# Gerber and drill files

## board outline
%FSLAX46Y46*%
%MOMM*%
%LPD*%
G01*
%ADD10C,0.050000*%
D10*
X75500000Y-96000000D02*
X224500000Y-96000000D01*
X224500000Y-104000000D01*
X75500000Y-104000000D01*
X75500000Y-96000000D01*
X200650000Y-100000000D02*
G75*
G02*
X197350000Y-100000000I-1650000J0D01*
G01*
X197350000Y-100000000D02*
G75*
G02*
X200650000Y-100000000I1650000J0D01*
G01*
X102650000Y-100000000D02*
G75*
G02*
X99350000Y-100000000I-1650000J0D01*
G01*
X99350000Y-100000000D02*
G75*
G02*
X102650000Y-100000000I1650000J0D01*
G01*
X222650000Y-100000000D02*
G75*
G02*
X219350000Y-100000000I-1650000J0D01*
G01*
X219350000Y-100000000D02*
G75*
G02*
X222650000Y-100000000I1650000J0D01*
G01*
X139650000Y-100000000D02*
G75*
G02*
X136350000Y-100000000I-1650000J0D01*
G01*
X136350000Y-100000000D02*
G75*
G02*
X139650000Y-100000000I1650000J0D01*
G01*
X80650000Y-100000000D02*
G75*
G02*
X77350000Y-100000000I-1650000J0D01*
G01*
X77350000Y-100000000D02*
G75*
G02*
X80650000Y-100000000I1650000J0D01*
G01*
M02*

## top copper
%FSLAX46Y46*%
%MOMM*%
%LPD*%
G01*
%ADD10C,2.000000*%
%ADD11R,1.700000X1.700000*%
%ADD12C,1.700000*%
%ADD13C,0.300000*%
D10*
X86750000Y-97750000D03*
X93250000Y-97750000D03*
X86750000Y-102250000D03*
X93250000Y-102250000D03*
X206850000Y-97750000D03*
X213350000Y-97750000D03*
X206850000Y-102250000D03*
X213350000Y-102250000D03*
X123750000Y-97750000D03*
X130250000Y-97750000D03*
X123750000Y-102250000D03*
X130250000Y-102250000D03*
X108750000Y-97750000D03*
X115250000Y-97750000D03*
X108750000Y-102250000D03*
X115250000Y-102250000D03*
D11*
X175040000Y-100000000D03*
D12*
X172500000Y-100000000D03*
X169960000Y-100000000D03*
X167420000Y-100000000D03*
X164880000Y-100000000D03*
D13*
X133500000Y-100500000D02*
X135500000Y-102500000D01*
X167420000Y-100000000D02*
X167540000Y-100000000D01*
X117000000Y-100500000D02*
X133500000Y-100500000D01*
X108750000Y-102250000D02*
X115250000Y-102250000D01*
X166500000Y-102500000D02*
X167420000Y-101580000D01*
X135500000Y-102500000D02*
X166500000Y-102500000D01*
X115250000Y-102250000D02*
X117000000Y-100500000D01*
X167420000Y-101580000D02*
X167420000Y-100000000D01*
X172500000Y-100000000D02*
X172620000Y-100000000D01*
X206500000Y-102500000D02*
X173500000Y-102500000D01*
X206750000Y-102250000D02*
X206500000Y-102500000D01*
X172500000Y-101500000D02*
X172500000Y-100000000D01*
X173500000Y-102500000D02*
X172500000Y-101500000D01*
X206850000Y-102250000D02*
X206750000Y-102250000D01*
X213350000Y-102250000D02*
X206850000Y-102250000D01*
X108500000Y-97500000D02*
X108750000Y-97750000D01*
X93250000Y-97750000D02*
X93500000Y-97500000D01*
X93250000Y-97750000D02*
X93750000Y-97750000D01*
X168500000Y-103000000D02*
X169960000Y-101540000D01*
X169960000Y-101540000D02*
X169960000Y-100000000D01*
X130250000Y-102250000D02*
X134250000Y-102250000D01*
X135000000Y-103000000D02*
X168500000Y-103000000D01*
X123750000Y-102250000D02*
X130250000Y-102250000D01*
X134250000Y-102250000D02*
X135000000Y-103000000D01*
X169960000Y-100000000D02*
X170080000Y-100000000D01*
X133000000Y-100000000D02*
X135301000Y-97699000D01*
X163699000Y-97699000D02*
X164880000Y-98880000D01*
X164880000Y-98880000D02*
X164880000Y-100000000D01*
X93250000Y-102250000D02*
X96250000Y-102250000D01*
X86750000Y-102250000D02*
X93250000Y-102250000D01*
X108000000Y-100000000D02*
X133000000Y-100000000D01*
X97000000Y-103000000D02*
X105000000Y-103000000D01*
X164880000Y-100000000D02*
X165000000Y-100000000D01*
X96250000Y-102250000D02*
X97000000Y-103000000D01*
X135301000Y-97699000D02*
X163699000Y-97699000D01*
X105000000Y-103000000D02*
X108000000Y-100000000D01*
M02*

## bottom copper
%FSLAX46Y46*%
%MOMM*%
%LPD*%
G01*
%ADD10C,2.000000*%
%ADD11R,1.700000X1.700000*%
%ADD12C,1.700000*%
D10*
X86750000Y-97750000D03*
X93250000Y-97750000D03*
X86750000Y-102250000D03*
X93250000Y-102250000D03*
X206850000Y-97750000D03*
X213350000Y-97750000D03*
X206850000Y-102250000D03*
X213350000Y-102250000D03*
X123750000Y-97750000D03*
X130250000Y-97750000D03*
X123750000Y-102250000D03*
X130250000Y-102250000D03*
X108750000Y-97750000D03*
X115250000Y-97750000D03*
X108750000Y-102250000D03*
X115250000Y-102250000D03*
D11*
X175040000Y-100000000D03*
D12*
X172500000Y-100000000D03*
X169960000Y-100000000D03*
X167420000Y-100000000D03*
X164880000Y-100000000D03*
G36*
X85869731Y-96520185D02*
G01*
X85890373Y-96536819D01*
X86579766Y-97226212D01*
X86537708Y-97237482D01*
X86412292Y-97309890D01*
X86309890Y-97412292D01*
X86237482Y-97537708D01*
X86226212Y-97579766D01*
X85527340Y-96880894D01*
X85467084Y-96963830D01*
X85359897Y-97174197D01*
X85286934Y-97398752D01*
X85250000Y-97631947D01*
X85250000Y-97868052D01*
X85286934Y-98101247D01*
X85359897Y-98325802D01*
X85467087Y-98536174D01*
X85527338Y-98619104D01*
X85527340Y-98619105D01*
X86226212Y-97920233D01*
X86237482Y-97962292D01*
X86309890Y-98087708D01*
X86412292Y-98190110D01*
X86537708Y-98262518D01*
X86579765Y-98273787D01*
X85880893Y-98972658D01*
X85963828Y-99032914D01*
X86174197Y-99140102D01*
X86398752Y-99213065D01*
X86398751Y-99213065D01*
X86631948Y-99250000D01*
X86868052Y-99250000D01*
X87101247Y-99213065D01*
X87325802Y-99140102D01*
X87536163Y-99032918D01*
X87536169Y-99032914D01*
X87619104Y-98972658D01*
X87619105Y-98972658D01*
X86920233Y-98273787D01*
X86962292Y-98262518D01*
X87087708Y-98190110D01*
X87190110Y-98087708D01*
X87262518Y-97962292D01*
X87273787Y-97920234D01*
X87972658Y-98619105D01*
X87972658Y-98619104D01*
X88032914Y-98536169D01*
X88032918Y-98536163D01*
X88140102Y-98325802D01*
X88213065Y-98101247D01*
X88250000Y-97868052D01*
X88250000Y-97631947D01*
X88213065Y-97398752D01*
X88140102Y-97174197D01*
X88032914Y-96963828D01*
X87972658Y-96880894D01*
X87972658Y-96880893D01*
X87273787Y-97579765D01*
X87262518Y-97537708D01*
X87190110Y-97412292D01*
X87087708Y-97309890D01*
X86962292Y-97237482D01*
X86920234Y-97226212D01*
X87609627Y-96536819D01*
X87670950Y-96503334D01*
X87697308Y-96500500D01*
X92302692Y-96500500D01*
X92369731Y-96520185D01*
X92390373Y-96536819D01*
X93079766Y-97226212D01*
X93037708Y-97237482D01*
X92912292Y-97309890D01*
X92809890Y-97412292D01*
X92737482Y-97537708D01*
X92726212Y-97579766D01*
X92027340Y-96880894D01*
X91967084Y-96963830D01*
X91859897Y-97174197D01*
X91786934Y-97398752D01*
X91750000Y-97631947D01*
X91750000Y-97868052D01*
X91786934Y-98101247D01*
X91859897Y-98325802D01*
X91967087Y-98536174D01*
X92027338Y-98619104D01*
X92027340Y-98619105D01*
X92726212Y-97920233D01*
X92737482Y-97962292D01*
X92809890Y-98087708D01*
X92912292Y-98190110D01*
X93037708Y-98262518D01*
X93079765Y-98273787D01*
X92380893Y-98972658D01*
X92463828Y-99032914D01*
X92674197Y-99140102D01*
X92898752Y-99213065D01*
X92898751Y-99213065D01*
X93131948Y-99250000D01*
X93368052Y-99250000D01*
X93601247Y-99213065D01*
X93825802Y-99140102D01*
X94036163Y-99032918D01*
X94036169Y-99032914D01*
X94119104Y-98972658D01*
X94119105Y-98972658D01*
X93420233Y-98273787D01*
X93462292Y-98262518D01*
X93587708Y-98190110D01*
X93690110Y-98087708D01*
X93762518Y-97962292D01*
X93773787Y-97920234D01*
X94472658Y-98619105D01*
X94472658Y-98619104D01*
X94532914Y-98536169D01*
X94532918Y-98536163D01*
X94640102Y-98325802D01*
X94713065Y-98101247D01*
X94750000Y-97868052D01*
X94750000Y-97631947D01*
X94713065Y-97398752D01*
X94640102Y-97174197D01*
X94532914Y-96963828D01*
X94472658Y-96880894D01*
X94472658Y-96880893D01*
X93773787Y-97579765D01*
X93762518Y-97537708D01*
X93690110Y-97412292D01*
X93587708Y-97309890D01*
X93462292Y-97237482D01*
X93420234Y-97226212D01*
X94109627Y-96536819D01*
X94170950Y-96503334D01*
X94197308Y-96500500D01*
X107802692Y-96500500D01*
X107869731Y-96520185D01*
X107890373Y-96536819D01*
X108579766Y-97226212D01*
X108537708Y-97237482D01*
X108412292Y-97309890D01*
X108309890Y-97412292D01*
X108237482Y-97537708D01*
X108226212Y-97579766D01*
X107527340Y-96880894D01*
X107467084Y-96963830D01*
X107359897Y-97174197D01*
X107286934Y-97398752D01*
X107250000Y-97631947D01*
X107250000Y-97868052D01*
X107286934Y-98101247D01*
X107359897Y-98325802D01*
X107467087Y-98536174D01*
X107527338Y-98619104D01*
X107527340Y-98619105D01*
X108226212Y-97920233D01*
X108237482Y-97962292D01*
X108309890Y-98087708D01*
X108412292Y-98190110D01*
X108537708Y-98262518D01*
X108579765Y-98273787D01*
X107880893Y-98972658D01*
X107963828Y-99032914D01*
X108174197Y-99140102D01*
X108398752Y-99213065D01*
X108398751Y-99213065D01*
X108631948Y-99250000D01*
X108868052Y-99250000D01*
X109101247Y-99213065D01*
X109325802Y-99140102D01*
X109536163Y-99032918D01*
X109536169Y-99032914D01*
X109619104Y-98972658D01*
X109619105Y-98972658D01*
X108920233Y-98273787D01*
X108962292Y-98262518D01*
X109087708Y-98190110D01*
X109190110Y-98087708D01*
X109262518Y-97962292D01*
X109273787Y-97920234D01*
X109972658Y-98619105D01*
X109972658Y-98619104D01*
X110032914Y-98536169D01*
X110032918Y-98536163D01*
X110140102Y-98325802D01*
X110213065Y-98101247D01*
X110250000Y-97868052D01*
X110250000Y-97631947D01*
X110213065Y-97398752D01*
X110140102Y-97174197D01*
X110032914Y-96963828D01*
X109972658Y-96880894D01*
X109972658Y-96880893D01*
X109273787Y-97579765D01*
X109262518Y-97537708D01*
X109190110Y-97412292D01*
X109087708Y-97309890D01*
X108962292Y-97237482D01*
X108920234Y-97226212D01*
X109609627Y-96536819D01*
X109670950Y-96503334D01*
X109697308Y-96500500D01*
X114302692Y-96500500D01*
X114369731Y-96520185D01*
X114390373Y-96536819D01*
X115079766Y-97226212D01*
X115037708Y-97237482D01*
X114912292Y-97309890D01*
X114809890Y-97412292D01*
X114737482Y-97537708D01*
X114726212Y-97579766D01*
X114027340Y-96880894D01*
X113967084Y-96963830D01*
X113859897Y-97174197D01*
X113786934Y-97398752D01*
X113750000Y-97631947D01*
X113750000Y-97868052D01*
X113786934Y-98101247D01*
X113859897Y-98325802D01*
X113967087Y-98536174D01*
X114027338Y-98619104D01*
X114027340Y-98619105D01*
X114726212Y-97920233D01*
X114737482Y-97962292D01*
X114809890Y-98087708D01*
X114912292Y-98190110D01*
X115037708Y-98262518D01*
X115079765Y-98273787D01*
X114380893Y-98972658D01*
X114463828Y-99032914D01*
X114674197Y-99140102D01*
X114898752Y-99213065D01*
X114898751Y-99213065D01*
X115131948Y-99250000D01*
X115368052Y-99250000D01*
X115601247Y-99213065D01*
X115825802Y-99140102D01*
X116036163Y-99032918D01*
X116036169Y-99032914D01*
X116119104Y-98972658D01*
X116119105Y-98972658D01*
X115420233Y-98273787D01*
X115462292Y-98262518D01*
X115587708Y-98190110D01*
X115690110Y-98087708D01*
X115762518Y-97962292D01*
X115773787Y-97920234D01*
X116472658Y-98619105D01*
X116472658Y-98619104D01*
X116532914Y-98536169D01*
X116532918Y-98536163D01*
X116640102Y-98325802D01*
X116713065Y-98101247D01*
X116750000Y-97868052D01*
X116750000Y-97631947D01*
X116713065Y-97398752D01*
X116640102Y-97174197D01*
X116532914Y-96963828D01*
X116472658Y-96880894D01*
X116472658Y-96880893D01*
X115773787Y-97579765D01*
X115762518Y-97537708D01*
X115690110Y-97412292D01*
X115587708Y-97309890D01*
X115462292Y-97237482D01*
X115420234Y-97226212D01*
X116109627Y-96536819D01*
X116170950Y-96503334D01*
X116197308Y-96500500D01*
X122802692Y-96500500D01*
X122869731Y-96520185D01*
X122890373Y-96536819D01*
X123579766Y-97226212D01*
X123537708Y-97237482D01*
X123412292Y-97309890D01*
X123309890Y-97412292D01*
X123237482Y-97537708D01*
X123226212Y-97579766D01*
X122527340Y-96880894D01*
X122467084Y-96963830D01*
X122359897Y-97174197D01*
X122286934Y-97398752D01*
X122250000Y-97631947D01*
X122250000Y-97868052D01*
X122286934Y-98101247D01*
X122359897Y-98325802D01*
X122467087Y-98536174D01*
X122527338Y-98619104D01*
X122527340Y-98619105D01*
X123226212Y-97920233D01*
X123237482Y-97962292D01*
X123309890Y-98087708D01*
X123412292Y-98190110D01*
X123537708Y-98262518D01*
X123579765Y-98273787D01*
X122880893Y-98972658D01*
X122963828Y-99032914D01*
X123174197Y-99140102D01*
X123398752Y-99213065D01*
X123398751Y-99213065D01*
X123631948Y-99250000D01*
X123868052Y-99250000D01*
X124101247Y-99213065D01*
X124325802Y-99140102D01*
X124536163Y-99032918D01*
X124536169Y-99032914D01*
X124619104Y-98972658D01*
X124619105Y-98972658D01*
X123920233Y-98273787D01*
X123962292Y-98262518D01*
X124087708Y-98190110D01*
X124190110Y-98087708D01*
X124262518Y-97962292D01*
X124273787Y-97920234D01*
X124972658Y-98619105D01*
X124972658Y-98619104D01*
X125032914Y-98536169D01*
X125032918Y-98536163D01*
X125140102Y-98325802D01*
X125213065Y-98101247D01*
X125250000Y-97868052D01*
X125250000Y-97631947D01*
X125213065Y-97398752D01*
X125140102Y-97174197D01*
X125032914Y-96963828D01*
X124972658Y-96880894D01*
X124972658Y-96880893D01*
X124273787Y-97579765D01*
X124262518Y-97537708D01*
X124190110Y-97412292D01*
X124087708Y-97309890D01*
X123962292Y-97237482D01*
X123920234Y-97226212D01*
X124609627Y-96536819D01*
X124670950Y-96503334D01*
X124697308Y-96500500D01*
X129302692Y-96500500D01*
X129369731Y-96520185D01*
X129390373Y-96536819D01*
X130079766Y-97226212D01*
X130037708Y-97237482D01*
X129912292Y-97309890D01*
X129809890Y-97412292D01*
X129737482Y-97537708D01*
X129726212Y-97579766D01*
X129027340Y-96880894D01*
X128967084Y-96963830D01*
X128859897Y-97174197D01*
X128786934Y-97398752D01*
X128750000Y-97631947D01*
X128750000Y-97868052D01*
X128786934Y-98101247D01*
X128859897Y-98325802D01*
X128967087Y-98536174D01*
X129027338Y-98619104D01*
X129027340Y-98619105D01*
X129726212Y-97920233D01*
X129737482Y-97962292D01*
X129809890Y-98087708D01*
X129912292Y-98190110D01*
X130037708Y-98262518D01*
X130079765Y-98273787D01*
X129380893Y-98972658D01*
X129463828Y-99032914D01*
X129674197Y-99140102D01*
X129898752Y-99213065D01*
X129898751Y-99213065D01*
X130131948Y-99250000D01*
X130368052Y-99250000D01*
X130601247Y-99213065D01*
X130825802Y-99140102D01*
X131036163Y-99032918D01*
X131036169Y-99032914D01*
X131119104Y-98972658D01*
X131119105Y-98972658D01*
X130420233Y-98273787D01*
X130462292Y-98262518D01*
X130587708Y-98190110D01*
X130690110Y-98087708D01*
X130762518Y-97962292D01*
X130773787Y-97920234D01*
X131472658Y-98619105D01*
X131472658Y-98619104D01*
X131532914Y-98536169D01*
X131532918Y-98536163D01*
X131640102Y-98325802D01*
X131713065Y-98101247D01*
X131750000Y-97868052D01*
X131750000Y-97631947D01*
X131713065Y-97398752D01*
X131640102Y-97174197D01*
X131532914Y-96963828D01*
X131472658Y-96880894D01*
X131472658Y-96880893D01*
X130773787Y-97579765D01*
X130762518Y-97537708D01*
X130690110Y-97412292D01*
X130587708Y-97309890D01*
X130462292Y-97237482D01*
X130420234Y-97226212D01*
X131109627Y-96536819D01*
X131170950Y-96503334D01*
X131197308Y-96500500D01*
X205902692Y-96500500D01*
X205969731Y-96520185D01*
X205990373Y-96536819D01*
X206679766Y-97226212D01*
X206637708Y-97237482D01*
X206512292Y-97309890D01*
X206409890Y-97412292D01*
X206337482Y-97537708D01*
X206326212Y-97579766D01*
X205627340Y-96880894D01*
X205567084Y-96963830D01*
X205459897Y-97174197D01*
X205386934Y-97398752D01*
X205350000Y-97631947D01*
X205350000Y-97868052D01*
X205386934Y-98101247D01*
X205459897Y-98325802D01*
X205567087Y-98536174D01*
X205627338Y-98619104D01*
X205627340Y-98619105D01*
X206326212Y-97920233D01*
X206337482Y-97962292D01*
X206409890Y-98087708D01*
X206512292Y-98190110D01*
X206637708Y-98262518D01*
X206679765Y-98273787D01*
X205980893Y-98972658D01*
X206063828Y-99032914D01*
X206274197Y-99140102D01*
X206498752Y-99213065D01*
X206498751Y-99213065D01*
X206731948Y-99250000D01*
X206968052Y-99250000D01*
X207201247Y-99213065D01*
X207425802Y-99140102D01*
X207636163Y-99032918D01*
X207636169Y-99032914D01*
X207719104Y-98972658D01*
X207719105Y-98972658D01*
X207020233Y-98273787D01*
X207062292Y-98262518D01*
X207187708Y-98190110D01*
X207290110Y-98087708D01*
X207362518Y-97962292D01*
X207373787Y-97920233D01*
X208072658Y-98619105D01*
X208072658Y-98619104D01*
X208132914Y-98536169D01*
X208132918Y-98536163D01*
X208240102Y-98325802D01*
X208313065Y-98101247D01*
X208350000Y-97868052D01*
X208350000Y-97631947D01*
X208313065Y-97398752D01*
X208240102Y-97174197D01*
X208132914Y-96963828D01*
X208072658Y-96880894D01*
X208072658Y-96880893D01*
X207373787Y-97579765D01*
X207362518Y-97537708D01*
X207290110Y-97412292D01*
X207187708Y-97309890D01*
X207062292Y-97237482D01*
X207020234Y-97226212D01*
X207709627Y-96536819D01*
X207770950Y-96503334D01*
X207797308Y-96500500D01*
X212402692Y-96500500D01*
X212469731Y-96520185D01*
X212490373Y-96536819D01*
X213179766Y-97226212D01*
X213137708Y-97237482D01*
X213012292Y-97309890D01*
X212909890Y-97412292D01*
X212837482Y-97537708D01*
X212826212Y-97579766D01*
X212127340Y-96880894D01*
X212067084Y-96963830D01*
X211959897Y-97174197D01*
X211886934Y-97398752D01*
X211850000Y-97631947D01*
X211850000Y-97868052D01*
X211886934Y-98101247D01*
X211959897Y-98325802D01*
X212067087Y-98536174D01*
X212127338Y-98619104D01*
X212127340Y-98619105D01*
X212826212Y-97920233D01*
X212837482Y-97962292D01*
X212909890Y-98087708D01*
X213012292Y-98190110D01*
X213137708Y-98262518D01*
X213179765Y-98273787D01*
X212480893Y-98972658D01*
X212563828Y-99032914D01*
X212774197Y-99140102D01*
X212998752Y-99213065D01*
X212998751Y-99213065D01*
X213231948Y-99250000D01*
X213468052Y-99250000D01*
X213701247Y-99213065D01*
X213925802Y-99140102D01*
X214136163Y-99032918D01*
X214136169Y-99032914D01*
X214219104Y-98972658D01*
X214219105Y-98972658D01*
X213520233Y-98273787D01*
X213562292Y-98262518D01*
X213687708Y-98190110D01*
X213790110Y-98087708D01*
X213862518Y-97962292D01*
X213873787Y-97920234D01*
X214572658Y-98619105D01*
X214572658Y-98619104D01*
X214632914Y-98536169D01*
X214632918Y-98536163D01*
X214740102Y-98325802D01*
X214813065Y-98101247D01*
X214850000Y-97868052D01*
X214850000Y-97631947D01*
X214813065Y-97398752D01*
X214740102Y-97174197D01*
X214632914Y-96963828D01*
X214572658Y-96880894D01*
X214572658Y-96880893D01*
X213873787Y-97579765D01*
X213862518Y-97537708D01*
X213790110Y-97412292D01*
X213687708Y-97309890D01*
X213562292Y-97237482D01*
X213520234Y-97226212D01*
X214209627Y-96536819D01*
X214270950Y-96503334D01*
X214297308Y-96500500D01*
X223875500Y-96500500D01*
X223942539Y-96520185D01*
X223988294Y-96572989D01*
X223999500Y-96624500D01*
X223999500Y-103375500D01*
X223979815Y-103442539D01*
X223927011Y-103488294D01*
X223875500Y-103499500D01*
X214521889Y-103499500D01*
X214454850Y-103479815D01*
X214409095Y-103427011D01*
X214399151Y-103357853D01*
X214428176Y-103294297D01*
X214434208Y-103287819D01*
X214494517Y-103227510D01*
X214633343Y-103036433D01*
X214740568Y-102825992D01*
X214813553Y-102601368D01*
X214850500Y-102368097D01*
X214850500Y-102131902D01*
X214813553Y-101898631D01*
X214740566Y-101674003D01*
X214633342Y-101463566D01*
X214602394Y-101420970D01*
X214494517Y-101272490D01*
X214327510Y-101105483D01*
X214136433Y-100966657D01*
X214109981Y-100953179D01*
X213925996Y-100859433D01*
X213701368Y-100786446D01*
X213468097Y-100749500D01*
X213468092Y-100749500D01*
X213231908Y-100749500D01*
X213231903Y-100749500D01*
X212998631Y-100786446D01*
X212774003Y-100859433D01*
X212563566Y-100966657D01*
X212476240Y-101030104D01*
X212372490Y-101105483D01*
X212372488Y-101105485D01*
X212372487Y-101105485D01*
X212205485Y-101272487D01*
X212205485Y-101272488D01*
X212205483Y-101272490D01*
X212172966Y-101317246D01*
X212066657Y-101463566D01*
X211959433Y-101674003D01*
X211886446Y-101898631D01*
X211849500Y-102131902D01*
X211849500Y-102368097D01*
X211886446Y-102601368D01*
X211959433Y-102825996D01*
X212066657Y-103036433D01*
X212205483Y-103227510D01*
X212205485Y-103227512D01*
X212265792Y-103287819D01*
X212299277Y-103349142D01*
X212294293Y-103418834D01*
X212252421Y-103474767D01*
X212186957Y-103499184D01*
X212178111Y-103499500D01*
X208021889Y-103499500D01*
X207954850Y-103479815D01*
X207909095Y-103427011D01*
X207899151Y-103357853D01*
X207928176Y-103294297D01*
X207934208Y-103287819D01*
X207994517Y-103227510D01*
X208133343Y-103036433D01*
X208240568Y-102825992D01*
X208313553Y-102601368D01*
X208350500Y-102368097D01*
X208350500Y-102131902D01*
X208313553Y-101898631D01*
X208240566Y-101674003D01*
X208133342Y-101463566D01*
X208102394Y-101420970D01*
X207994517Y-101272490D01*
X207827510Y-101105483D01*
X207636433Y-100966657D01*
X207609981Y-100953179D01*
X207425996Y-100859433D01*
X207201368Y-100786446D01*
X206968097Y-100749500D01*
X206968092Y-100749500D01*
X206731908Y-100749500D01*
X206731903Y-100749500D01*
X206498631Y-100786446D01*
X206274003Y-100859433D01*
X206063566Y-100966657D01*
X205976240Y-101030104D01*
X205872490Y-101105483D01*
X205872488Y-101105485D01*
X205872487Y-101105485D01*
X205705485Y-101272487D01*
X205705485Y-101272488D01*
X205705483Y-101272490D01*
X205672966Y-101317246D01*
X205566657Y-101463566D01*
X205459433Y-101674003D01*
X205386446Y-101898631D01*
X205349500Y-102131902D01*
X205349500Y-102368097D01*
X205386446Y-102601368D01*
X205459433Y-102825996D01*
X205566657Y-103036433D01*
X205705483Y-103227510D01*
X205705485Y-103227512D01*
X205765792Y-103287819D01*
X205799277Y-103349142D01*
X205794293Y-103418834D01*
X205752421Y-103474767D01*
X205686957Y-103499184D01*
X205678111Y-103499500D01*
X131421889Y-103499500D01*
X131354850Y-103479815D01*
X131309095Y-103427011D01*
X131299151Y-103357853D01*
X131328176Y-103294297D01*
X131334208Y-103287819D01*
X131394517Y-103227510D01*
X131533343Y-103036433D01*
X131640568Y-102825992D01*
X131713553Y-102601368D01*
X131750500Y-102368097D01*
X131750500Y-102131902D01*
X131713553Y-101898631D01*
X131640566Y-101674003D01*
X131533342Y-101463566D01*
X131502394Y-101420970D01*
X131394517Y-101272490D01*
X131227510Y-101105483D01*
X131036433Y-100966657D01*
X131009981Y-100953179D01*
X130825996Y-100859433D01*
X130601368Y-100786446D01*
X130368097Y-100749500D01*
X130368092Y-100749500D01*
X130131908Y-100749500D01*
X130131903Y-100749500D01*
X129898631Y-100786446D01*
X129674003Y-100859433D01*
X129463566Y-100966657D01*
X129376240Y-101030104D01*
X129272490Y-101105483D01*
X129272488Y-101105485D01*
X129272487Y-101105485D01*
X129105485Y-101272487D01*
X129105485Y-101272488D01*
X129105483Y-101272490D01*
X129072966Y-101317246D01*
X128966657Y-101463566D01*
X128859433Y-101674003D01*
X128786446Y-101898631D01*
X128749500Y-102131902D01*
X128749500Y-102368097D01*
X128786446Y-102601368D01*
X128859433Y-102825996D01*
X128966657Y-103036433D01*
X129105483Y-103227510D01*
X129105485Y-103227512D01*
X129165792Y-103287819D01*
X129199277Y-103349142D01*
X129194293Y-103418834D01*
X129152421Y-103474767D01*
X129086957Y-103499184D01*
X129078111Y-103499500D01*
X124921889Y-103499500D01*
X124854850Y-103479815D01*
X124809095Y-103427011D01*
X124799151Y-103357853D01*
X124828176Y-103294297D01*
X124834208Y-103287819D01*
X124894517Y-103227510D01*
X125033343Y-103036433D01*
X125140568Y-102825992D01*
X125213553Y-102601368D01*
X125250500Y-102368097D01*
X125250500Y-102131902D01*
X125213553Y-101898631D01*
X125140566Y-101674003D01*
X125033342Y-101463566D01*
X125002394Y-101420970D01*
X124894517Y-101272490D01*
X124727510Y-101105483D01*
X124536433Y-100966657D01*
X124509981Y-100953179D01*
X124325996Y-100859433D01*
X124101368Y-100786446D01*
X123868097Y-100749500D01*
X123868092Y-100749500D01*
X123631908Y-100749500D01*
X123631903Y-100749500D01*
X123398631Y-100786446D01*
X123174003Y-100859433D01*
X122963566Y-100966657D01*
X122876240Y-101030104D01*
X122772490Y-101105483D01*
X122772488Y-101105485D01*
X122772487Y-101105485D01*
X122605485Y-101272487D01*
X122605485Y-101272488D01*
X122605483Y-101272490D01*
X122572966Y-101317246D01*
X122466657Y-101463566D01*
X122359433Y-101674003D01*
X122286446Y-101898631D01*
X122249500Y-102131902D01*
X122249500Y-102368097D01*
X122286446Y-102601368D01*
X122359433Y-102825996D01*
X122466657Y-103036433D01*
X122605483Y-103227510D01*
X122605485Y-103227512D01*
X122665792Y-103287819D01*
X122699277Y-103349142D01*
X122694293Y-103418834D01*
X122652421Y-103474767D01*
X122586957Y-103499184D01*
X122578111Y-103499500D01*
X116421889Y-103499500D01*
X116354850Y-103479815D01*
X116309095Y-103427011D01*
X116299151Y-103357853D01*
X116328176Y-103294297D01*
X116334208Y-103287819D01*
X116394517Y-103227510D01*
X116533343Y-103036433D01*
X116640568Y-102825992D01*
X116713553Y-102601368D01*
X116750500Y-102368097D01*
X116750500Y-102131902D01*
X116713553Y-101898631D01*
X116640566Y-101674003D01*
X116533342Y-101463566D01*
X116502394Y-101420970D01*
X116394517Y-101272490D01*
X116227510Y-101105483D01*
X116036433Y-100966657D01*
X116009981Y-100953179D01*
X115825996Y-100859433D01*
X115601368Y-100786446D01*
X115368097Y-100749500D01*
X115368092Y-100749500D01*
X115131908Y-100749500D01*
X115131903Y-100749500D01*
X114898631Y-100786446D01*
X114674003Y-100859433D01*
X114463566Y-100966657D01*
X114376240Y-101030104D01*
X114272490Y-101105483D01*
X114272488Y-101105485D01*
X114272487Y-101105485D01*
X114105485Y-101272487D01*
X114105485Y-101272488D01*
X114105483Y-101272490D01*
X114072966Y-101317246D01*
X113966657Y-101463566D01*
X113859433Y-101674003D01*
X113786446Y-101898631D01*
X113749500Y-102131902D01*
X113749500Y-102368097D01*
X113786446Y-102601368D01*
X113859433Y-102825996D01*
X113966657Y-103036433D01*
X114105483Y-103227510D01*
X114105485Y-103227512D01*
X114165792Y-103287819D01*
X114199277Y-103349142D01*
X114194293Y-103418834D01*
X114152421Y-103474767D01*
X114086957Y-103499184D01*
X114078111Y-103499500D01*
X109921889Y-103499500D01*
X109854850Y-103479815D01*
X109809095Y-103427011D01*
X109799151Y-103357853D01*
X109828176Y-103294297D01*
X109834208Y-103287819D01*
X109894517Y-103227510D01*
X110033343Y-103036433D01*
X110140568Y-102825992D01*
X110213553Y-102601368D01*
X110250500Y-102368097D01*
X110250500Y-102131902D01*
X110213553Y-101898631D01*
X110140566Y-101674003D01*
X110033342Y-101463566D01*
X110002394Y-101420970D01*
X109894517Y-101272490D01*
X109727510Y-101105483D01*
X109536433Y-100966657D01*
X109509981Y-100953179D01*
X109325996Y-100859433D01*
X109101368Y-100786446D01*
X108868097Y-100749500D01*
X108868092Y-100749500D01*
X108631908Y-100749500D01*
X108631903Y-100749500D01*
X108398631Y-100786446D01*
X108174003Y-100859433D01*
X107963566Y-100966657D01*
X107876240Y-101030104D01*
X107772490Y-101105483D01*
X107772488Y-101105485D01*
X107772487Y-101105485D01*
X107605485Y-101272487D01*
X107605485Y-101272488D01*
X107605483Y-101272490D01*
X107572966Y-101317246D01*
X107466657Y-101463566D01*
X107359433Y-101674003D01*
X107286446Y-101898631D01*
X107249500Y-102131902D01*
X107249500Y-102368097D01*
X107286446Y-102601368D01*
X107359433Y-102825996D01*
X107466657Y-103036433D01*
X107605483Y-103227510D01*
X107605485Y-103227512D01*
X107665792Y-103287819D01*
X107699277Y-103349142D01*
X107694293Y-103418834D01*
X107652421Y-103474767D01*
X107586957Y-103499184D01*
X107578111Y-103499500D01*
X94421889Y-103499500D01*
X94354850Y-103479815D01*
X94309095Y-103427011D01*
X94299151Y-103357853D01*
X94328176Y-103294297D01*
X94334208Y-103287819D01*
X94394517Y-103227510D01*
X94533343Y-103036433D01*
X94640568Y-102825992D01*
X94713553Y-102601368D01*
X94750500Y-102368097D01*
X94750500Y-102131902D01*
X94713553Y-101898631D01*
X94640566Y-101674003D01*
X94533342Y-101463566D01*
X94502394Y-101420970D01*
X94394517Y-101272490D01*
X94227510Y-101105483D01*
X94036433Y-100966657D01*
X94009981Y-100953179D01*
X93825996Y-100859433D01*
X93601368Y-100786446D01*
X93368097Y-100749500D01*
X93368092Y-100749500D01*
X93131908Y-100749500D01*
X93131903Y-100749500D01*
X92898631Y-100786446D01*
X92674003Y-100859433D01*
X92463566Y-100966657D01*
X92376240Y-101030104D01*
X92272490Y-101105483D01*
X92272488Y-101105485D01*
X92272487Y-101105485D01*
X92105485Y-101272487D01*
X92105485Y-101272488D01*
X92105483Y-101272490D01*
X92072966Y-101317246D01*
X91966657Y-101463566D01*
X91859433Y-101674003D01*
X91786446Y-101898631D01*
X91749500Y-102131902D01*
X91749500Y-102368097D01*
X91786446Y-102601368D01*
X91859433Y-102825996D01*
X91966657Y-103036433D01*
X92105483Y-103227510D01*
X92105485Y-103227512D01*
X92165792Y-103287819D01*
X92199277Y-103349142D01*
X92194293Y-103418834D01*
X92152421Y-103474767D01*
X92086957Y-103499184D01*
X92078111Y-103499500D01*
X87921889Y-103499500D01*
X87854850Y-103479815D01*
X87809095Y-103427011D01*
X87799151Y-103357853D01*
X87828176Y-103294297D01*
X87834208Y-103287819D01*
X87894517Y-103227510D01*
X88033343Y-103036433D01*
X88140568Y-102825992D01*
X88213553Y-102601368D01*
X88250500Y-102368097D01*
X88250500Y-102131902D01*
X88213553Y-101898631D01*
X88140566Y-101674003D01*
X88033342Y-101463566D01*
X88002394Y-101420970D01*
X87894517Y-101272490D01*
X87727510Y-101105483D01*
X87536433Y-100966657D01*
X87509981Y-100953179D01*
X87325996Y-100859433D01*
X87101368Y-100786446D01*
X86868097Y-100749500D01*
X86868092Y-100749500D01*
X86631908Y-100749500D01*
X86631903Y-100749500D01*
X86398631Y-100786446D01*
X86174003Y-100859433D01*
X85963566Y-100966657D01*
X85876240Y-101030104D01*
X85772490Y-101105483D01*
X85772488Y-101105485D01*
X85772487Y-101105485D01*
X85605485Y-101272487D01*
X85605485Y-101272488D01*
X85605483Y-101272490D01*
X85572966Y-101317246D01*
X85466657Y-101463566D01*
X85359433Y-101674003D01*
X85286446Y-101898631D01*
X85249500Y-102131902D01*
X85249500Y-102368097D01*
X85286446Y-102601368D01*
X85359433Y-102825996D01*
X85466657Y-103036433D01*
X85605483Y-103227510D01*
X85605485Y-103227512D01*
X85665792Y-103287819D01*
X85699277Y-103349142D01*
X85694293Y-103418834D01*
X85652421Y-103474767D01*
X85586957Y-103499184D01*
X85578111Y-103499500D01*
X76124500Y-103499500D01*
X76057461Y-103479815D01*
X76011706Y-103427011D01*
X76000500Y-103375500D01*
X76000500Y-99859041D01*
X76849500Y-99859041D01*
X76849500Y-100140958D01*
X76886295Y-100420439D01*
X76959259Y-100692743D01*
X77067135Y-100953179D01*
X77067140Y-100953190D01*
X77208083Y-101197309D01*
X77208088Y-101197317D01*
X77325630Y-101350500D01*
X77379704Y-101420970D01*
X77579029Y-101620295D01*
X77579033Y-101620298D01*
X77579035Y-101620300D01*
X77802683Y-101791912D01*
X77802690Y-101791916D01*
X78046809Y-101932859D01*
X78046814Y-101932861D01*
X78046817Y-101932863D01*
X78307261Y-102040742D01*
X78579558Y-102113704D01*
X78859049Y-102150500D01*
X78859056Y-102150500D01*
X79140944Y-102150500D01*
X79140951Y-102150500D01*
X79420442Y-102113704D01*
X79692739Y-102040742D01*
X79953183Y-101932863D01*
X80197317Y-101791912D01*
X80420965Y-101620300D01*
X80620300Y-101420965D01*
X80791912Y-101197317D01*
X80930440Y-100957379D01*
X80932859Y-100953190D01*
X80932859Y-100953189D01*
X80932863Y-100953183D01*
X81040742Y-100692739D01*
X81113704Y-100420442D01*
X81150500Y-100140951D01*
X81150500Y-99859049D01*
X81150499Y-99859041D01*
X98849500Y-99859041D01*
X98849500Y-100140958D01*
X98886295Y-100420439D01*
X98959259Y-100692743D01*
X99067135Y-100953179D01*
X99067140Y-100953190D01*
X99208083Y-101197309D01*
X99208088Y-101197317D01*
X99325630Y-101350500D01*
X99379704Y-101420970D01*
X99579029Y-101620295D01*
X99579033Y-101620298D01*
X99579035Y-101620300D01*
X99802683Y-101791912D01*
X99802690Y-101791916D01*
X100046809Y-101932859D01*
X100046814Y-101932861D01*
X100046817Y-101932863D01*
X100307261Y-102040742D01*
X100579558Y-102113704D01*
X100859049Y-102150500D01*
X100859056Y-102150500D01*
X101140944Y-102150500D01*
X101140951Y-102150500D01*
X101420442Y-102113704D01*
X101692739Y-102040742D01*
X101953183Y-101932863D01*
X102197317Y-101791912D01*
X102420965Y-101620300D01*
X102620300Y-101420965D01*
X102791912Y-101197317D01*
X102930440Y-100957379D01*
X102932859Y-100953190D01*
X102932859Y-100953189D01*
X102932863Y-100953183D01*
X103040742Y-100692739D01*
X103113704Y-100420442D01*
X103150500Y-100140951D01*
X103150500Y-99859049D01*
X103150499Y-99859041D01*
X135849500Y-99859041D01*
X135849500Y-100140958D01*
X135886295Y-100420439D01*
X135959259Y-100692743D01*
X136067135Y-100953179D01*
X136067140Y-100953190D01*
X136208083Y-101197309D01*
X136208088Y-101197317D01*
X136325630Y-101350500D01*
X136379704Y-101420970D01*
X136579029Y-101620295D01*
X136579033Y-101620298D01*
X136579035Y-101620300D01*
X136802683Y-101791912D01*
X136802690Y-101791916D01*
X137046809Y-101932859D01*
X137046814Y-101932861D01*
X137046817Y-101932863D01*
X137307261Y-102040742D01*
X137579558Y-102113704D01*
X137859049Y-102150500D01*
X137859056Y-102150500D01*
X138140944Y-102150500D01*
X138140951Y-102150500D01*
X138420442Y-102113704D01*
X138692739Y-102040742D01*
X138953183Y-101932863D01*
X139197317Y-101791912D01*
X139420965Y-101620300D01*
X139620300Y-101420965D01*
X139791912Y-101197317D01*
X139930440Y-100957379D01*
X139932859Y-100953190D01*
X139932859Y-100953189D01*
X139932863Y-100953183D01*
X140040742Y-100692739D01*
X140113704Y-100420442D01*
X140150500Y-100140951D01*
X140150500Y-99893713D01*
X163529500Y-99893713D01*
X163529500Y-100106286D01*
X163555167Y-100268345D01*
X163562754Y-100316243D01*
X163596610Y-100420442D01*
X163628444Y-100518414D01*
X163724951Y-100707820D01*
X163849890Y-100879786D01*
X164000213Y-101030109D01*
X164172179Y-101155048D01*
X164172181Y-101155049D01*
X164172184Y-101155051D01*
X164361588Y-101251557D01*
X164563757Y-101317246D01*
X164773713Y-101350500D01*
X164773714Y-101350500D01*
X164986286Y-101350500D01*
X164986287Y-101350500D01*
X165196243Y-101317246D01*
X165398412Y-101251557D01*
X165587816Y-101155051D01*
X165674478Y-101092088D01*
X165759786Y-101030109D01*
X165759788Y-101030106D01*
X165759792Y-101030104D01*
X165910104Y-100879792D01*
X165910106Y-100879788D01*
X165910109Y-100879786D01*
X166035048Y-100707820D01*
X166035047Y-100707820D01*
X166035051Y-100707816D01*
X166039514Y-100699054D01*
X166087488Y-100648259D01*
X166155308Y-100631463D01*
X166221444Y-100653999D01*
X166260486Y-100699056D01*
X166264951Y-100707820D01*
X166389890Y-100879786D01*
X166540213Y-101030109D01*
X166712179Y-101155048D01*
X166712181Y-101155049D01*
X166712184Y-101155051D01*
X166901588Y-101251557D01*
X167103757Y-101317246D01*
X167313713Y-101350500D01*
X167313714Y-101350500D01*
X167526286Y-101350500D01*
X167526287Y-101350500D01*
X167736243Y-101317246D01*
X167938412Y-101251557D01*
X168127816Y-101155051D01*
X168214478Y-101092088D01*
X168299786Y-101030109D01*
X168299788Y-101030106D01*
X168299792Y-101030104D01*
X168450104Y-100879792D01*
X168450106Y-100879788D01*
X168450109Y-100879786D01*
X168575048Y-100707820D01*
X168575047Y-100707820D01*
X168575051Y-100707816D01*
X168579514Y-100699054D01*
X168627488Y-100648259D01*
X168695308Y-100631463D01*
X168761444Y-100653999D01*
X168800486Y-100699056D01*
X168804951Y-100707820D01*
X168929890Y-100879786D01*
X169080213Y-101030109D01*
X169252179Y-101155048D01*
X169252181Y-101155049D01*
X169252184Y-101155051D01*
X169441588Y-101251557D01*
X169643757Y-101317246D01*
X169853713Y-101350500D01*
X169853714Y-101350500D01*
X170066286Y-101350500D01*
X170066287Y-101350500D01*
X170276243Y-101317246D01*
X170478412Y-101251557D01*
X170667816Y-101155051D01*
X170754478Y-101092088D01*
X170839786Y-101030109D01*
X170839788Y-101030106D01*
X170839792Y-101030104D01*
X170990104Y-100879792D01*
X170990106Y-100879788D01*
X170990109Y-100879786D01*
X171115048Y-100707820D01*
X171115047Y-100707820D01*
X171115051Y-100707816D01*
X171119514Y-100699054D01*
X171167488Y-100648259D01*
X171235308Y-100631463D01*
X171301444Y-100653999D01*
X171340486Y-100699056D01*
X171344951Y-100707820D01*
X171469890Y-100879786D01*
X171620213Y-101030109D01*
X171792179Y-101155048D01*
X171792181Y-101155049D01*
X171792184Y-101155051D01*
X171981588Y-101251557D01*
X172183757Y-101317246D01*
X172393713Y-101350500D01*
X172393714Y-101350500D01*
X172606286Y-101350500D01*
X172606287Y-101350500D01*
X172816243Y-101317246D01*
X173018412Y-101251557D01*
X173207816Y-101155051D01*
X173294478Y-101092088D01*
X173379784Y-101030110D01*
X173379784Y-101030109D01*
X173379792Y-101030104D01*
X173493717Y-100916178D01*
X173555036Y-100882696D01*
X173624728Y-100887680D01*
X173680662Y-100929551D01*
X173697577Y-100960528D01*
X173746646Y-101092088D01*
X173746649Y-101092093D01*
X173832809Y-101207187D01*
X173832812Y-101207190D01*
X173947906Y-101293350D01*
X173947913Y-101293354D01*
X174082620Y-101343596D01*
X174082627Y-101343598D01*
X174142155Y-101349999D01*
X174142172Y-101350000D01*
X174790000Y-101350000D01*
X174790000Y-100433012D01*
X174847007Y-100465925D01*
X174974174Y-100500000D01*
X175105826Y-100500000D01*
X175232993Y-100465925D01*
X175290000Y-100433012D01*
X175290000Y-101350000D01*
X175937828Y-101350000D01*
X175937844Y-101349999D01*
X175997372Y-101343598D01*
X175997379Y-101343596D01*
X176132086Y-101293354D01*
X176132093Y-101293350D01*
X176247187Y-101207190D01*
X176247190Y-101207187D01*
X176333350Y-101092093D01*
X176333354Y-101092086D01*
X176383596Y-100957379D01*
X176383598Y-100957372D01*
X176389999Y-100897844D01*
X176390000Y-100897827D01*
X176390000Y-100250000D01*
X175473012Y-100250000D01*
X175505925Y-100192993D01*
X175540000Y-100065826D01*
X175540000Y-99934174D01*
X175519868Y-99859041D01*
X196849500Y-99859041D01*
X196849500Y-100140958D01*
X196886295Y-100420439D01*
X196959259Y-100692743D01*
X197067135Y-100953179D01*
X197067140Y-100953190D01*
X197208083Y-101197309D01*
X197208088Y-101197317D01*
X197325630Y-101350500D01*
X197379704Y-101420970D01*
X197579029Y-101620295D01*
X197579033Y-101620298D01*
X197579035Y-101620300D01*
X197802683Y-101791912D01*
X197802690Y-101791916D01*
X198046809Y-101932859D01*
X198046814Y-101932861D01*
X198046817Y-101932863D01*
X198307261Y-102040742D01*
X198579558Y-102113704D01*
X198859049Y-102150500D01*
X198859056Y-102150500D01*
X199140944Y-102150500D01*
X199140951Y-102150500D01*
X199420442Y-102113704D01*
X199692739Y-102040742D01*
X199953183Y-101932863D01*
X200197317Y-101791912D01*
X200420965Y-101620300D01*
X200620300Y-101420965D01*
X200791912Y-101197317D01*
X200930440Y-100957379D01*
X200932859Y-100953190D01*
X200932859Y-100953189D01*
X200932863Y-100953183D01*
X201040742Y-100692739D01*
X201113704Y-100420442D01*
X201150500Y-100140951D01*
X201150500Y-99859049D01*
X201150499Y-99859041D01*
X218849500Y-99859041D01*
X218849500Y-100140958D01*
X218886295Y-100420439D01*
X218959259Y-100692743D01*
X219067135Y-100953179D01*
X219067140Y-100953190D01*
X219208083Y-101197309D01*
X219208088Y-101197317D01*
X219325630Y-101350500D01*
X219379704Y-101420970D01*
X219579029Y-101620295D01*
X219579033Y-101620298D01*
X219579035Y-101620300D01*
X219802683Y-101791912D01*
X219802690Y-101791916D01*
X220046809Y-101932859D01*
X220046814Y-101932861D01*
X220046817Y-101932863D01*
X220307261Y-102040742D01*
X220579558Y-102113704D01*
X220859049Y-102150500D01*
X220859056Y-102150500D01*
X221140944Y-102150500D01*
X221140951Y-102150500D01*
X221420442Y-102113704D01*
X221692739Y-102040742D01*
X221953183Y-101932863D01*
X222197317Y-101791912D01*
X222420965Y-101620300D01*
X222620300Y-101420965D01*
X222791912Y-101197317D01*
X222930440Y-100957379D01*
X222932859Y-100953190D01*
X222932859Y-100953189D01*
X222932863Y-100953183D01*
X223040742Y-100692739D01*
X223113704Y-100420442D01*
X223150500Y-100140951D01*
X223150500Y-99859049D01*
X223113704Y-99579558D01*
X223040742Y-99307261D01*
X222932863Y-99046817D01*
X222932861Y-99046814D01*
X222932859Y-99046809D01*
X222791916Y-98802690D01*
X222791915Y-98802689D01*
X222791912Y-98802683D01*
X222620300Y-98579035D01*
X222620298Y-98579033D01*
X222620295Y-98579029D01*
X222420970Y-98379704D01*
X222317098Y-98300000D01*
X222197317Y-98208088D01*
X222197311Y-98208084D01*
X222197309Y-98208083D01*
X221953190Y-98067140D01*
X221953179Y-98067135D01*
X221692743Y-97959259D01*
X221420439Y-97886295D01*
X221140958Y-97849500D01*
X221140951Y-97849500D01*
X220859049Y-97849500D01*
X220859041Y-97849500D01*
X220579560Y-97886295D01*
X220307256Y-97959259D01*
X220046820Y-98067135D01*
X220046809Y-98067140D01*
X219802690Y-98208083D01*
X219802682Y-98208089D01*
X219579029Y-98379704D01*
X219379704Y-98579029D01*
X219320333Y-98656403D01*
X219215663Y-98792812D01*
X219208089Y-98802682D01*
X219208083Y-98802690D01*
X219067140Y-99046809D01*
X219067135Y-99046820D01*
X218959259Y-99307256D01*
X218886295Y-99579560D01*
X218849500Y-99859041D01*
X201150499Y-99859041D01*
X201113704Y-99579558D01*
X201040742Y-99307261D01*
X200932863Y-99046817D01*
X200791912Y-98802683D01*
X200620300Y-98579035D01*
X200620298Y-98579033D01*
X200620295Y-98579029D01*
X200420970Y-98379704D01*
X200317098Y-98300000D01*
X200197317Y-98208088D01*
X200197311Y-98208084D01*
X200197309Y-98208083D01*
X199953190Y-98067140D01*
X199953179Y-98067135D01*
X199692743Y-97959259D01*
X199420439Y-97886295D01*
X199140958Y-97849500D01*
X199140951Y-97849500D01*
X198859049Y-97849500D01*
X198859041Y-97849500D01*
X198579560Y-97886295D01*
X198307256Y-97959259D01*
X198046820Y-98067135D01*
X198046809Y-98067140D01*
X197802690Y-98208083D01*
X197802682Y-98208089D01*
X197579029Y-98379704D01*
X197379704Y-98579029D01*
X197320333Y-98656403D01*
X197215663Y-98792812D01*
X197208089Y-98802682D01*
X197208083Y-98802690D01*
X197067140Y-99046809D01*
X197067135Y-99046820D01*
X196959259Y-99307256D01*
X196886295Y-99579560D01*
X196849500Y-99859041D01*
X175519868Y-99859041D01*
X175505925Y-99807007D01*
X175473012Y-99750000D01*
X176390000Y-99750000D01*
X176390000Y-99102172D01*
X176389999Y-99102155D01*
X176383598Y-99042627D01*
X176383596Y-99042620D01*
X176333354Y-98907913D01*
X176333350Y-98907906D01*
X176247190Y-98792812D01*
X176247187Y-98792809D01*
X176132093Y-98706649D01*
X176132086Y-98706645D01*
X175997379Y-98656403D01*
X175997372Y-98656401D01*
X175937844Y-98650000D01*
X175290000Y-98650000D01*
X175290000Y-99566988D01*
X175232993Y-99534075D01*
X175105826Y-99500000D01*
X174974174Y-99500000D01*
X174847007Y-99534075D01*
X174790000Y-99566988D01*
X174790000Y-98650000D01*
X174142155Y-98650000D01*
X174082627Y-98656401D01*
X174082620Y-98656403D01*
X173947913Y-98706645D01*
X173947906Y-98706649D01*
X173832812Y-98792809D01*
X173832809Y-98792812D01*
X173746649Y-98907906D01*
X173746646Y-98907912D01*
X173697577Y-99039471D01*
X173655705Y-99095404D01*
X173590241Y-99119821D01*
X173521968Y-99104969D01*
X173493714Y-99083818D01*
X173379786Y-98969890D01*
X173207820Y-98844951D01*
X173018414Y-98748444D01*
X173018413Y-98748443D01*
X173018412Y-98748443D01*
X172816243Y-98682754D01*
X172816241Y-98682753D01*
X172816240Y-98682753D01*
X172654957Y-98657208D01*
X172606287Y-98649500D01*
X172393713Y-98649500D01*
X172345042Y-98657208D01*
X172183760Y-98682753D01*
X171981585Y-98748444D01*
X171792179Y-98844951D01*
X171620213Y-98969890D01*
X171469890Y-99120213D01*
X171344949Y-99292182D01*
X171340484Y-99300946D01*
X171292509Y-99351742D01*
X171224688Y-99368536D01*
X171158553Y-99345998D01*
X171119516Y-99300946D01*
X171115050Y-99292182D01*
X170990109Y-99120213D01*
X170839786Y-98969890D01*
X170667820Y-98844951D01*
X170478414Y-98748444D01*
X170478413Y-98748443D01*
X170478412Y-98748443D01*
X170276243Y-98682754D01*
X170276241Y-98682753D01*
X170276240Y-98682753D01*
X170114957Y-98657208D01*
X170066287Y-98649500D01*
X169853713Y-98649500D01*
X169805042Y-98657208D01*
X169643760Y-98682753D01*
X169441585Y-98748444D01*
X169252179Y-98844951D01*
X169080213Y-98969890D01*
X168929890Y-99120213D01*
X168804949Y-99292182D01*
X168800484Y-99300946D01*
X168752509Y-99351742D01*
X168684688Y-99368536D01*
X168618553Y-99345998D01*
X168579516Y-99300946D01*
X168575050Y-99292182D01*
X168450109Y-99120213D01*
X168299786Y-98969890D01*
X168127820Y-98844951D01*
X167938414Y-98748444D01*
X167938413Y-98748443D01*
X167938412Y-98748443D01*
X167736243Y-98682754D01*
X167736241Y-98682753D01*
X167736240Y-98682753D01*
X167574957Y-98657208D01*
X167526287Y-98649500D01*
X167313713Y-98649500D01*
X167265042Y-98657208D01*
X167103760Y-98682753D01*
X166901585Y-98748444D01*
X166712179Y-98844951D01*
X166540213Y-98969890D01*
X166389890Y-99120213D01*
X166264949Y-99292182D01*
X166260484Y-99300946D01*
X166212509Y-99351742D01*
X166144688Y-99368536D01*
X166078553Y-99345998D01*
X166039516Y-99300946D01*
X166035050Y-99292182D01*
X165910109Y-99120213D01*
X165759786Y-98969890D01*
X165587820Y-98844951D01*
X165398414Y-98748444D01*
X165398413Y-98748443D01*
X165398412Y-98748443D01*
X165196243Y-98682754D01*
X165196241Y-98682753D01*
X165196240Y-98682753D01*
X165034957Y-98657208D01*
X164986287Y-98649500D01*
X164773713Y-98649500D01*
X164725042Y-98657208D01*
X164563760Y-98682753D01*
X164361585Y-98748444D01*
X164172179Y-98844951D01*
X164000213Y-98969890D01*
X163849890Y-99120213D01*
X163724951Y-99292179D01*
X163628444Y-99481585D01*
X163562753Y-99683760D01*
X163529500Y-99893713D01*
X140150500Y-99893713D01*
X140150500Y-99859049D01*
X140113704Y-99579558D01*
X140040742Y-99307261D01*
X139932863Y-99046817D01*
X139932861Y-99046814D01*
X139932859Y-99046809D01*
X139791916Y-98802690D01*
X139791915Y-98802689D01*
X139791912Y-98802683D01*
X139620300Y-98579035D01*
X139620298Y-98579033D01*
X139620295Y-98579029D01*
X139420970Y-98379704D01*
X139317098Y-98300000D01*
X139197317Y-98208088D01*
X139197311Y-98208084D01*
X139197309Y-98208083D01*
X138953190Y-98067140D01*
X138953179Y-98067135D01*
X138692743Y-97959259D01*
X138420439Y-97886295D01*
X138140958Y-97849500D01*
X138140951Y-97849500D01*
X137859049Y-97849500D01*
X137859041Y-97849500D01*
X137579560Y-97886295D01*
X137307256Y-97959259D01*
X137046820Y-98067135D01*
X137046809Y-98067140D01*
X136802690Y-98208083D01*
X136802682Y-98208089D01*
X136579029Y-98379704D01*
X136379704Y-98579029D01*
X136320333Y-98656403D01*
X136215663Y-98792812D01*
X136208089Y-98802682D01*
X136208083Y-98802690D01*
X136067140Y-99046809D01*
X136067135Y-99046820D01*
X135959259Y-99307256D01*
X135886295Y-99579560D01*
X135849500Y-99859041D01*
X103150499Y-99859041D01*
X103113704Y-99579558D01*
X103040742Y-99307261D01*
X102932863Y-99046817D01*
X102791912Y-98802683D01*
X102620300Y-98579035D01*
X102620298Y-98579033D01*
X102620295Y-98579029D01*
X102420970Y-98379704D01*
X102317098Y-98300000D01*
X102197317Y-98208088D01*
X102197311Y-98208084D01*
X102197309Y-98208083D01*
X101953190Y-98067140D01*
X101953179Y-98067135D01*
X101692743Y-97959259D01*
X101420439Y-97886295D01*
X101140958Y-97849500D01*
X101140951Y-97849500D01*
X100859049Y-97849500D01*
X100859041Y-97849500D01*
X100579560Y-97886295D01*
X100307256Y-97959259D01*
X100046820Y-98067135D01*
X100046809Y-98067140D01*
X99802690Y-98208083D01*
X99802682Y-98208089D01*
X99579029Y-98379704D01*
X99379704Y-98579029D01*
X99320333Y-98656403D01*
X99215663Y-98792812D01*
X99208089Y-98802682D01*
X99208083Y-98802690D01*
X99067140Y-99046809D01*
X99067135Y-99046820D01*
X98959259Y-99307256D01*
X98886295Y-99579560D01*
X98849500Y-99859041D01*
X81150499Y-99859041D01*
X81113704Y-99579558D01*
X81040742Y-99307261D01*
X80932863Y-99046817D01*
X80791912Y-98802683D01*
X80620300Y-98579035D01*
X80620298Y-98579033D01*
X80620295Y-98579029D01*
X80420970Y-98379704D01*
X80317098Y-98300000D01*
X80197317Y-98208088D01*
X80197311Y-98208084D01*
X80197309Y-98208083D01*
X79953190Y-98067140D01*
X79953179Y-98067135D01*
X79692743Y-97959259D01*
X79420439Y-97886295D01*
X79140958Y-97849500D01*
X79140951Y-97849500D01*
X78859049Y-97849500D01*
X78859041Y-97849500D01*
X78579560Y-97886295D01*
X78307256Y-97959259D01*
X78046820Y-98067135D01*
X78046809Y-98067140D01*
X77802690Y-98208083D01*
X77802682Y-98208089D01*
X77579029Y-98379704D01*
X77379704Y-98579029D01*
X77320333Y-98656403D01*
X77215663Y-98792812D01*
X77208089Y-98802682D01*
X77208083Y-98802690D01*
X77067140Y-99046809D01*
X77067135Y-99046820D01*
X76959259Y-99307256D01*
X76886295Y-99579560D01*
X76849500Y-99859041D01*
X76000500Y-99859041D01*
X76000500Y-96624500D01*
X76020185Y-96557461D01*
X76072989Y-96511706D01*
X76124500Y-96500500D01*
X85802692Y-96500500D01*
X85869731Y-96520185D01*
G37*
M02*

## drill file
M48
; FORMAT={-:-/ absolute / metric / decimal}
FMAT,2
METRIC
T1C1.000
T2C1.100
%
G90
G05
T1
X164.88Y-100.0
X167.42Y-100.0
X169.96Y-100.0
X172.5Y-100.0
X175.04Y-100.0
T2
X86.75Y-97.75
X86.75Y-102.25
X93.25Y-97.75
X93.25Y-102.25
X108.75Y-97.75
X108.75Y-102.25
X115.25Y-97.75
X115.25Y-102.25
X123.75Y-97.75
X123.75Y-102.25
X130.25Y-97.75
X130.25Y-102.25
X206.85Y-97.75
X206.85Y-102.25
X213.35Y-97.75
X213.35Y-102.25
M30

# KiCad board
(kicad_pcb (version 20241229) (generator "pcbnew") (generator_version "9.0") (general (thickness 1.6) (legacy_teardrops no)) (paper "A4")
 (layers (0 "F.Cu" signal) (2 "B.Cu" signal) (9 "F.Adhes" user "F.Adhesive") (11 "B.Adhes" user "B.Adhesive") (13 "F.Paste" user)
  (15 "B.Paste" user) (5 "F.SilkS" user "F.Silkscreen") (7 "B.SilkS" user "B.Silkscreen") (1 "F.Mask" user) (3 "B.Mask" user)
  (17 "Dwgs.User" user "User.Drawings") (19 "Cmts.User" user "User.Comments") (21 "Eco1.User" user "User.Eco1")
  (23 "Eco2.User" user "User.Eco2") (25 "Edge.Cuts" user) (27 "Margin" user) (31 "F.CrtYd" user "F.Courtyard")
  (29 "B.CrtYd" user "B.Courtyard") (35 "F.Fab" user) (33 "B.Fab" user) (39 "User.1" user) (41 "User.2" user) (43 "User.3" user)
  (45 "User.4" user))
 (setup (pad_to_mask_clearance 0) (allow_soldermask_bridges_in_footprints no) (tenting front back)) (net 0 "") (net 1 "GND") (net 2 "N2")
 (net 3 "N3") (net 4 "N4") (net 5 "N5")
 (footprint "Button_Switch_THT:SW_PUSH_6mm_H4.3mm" (layer "F.Cu") (at 86.75 97.75)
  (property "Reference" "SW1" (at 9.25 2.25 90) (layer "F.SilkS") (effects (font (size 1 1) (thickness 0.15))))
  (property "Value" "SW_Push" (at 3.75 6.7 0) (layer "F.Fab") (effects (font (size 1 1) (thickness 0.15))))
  (pad "1" thru_hole circle (at 0 0 90) (size 2 2) (drill 1.1) (layers "*.Cu" "*.Mask") (remove_unused_layers no) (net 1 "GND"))
  (pad "1" thru_hole circle (at 6.5 0 90) (size 2 2) (drill 1.1) (layers "*.Cu" "*.Mask") (remove_unused_layers no) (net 1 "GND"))
  (pad "2" thru_hole circle (at 0 4.5 90) (size 2 2) (drill 1.1) (layers "*.Cu" "*.Mask") (remove_unused_layers no) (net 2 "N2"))
  (pad "2" thru_hole circle (at 6.5 4.5 90) (size 2 2) (drill 1.1) (layers "*.Cu" "*.Mask") (remove_unused_layers no) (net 2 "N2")))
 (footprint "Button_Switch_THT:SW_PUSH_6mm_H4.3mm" (layer "F.Cu") (at 206.85 97.75)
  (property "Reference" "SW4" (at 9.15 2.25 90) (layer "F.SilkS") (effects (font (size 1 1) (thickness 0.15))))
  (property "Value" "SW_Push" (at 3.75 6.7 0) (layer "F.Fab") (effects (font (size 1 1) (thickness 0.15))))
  (pad "1" thru_hole circle (at 0 0 90) (size 2 2) (drill 1.1) (layers "*.Cu" "*.Mask") (remove_unused_layers no) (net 1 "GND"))
  (pad "1" thru_hole circle (at 6.5 0 90) (size 2 2) (drill 1.1) (layers "*.Cu" "*.Mask") (remove_unused_layers no) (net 1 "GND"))
  (pad "2" thru_hole circle (at 0 4.5 90) (size 2 2) (drill 1.1) (layers "*.Cu" "*.Mask") (remove_unused_layers no) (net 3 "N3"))
  (pad "2" thru_hole circle (at 6.5 4.5 90) (size 2 2) (drill 1.1) (layers "*.Cu" "*.Mask") (remove_unused_layers no) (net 3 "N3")))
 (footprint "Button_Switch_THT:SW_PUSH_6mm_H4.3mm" (layer "F.Cu") (at 123.75 97.75)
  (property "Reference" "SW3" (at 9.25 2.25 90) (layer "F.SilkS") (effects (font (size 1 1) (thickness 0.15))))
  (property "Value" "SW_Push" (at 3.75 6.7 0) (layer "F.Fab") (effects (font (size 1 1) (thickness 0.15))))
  (pad "1" thru_hole circle (at 0 0 90) (size 2 2) (drill 1.1) (layers "*.Cu" "*.Mask") (remove_unused_layers no) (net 1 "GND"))
  (pad "1" thru_hole circle (at 6.5 0 90) (size 2 2) (drill 1.1) (layers "*.Cu" "*.Mask") (remove_unused_layers no) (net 1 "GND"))
  (pad "2" thru_hole circle (at 0 4.5 90) (size 2 2) (drill 1.1) (layers "*.Cu" "*.Mask") (remove_unused_layers no) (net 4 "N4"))
  (pad "2" thru_hole circle (at 6.5 4.5 90) (size 2 2) (drill 1.1) (layers "*.Cu" "*.Mask") (remove_unused_layers no) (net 4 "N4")))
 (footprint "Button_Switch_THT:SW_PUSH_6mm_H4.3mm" (layer "F.Cu") (at 108.75 97.75)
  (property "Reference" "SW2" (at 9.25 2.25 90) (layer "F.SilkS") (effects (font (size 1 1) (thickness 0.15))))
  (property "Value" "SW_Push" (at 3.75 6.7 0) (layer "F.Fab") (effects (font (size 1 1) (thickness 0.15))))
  (pad "1" thru_hole circle (at 0 0 90) (size 2 2) (drill 1.1) (layers "*.Cu" "*.Mask") (remove_unused_layers no) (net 1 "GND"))
  (pad "1" thru_hole circle (at 6.5 0 90) (size 2 2) (drill 1.1) (layers "*.Cu" "*.Mask") (remove_unused_layers no) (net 1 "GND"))
  (pad "2" thru_hole circle (at 0 4.5 90) (size 2 2) (drill 1.1) (layers "*.Cu" "*.Mask") (remove_unused_layers no) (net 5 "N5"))
  (pad "2" thru_hole circle (at 6.5 4.5 90) (size 2 2) (drill 1.1) (layers "*.Cu" "*.Mask") (remove_unused_layers no) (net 5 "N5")))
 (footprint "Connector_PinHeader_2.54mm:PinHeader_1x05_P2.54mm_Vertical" (layer "B.Cu") (at 175.04 100 90)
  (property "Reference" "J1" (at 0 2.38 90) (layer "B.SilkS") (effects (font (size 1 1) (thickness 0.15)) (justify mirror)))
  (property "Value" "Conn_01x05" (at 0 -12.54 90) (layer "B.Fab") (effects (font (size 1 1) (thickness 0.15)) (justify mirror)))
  (pad "1" thru_hole rect (at 0 0 90) (size 1.7 1.7) (drill 1) (layers "*.Cu" "*.Mask") (remove_unused_layers no) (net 1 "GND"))
  (pad "2" thru_hole circle (at 0 -2.54 90) (size 1.7 1.7) (drill 1) (layers "*.Cu" "*.Mask") (remove_unused_layers no) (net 3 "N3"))
  (pad "3" thru_hole circle (at 0 -5.08 90) (size 1.7 1.7) (drill 1) (layers "*.Cu" "*.Mask") (remove_unused_layers no) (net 4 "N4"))
  (pad "4" thru_hole circle (at 0 -7.62 90) (size 1.7 1.7) (drill 1) (layers "*.Cu" "*.Mask") (remove_unused_layers no) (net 5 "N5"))
  (pad "5" thru_hole circle (at 0 -10.16 90) (size 1.7 1.7) (drill 1) (layers "*.Cu" "*.Mask") (remove_unused_layers no) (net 2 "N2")))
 (gr_rect (start 75.5 96) (end 224.5 104) (stroke (width 0.05) (type solid)) (fill no) (layer "Edge.Cuts"))
 (gr_circle (center 199 100) (end 200.65 100) (stroke (width 0.05) (type solid)) (fill no) (layer "Edge.Cuts"))
 (gr_circle (center 101 100) (end 102.65 100) (stroke (width 0.05) (type solid)) (fill no) (layer "Edge.Cuts"))
 (gr_circle (center 221 100) (end 222.65 100) (stroke (width 0.05) (type solid)) (fill no) (layer "Edge.Cuts"))
 (gr_circle (center 138 100) (end 139.65 100) (stroke (width 0.05) (type solid)) (fill no) (layer "Edge.Cuts"))
 (gr_circle (center 79 100) (end 80.65 100) (stroke (width 0.05) (type solid)) (fill no) (layer "Edge.Cuts"))
 (segment (start 133.5 100.5) (end 135.5 102.5) (width 0.3) (layer "F.Cu") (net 5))
 (segment (start 167.42 100) (end 167.54 100) (width 0.3) (layer "F.Cu") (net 5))
 (segment (start 117 100.5) (end 133.5 100.5) (width 0.3) (layer "F.Cu") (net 5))
 (segment (start 108.75 102.25) (end 115.25 102.25) (width 0.3) (layer "F.Cu") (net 5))
 (segment (start 166.5 102.5) (end 167.42 101.58) (width 0.3) (layer "F.Cu") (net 5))
 (segment (start 135.5 102.5) (end 166.5 102.5) (width 0.3) (layer "F.Cu") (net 5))
 (segment (start 115.25 102.25) (end 117 100.5) (width 0.3) (layer "F.Cu") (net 5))
 (segment (start 167.42 101.58) (end 167.42 100) (width 0.3) (layer "F.Cu") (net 5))
 (segment (start 172.5 100) (end 172.62 100) (width 0.3) (layer "F.Cu") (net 3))
 (segment (start 206.5 102.5) (end 173.5 102.5) (width 0.3) (layer "F.Cu") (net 3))
 (segment (start 206.75 102.25) (end 206.5 102.5) (width 0.3) (layer "F.Cu") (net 3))
 (segment (start 172.5 101.5) (end 172.5 100) (width 0.3) (layer "F.Cu") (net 3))
 (segment (start 173.5 102.5) (end 172.5 101.5) (width 0.3) (layer "F.Cu") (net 3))
 (segment (start 206.85 102.25) (end 206.75 102.25) (width 0.3) (layer "F.Cu") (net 3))
 (segment (start 213.35 102.25) (end 206.85 102.25) (width 0.3) (layer "F.Cu") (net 3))
 (segment (start 108.5 97.5) (end 108.75 97.75) (width 0.3) (layer "F.Cu") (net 1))
 (segment (start 93.25 97.75) (end 93.5 97.5) (width 0.3) (layer "F.Cu") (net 1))
 (segment (start 93.25 97.75) (end 93.75 97.75) (width 0.3) (layer "F.Cu") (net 1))
 (segment (start 168.5 103) (end 169.96 101.54) (width 0.3) (layer "F.Cu") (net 4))
 (segment (start 169.96 101.54) (end 169.96 100) (width 0.3) (layer "F.Cu") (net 4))
 (segment (start 130.25 102.25) (end 134.25 102.25) (width 0.3) (layer "F.Cu") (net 4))
 (segment (start 135 103) (end 168.5 103) (width 0.3) (layer "F.Cu") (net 4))
 (segment (start 123.75 102.25) (end 130.25 102.25) (width 0.3) (layer "F.Cu") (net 4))
 (segment (start 134.25 102.25) (end 135 103) (width 0.3) (layer "F.Cu") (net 4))
 (segment (start 169.96 100) (end 170.08 100) (width 0.3) (layer "F.Cu") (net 4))
 (segment (start 133 100) (end 135.301 97.699) (width 0.3) (layer "F.Cu") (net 2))
 (segment (start 163.699 97.699) (end 164.88 98.88) (width 0.3) (layer "F.Cu") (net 2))
 (segment (start 164.88 98.88) (end 164.88 100) (width 0.3) (layer "F.Cu") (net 2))
 (segment (start 93.25 102.25) (end 96.25 102.25) (width 0.3) (layer "F.Cu") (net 2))
 (segment (start 86.75 102.25) (end 93.25 102.25) (width 0.3) (layer "F.Cu") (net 2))
 (segment (start 108 100) (end 133 100) (width 0.3) (layer "F.Cu") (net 2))
 (segment (start 97 103) (end 105 103) (width 0.3) (layer "F.Cu") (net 2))
 (segment (start 164.88 100) (end 165 100) (width 0.3) (layer "F.Cu") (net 2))
 (segment (start 96.25 102.25) (end 97 103) (width 0.3) (layer "F.Cu") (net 2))
 (segment (start 135.301 97.699) (end 163.699 97.699) (width 0.3) (layer "F.Cu") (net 2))
 (segment (start 105 103) (end 108 100) (width 0.3) (layer "F.Cu") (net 2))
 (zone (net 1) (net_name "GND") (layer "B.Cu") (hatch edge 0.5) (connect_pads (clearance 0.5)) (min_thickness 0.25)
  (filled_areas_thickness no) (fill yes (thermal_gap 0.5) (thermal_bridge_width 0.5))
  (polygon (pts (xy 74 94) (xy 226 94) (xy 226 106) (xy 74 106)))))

